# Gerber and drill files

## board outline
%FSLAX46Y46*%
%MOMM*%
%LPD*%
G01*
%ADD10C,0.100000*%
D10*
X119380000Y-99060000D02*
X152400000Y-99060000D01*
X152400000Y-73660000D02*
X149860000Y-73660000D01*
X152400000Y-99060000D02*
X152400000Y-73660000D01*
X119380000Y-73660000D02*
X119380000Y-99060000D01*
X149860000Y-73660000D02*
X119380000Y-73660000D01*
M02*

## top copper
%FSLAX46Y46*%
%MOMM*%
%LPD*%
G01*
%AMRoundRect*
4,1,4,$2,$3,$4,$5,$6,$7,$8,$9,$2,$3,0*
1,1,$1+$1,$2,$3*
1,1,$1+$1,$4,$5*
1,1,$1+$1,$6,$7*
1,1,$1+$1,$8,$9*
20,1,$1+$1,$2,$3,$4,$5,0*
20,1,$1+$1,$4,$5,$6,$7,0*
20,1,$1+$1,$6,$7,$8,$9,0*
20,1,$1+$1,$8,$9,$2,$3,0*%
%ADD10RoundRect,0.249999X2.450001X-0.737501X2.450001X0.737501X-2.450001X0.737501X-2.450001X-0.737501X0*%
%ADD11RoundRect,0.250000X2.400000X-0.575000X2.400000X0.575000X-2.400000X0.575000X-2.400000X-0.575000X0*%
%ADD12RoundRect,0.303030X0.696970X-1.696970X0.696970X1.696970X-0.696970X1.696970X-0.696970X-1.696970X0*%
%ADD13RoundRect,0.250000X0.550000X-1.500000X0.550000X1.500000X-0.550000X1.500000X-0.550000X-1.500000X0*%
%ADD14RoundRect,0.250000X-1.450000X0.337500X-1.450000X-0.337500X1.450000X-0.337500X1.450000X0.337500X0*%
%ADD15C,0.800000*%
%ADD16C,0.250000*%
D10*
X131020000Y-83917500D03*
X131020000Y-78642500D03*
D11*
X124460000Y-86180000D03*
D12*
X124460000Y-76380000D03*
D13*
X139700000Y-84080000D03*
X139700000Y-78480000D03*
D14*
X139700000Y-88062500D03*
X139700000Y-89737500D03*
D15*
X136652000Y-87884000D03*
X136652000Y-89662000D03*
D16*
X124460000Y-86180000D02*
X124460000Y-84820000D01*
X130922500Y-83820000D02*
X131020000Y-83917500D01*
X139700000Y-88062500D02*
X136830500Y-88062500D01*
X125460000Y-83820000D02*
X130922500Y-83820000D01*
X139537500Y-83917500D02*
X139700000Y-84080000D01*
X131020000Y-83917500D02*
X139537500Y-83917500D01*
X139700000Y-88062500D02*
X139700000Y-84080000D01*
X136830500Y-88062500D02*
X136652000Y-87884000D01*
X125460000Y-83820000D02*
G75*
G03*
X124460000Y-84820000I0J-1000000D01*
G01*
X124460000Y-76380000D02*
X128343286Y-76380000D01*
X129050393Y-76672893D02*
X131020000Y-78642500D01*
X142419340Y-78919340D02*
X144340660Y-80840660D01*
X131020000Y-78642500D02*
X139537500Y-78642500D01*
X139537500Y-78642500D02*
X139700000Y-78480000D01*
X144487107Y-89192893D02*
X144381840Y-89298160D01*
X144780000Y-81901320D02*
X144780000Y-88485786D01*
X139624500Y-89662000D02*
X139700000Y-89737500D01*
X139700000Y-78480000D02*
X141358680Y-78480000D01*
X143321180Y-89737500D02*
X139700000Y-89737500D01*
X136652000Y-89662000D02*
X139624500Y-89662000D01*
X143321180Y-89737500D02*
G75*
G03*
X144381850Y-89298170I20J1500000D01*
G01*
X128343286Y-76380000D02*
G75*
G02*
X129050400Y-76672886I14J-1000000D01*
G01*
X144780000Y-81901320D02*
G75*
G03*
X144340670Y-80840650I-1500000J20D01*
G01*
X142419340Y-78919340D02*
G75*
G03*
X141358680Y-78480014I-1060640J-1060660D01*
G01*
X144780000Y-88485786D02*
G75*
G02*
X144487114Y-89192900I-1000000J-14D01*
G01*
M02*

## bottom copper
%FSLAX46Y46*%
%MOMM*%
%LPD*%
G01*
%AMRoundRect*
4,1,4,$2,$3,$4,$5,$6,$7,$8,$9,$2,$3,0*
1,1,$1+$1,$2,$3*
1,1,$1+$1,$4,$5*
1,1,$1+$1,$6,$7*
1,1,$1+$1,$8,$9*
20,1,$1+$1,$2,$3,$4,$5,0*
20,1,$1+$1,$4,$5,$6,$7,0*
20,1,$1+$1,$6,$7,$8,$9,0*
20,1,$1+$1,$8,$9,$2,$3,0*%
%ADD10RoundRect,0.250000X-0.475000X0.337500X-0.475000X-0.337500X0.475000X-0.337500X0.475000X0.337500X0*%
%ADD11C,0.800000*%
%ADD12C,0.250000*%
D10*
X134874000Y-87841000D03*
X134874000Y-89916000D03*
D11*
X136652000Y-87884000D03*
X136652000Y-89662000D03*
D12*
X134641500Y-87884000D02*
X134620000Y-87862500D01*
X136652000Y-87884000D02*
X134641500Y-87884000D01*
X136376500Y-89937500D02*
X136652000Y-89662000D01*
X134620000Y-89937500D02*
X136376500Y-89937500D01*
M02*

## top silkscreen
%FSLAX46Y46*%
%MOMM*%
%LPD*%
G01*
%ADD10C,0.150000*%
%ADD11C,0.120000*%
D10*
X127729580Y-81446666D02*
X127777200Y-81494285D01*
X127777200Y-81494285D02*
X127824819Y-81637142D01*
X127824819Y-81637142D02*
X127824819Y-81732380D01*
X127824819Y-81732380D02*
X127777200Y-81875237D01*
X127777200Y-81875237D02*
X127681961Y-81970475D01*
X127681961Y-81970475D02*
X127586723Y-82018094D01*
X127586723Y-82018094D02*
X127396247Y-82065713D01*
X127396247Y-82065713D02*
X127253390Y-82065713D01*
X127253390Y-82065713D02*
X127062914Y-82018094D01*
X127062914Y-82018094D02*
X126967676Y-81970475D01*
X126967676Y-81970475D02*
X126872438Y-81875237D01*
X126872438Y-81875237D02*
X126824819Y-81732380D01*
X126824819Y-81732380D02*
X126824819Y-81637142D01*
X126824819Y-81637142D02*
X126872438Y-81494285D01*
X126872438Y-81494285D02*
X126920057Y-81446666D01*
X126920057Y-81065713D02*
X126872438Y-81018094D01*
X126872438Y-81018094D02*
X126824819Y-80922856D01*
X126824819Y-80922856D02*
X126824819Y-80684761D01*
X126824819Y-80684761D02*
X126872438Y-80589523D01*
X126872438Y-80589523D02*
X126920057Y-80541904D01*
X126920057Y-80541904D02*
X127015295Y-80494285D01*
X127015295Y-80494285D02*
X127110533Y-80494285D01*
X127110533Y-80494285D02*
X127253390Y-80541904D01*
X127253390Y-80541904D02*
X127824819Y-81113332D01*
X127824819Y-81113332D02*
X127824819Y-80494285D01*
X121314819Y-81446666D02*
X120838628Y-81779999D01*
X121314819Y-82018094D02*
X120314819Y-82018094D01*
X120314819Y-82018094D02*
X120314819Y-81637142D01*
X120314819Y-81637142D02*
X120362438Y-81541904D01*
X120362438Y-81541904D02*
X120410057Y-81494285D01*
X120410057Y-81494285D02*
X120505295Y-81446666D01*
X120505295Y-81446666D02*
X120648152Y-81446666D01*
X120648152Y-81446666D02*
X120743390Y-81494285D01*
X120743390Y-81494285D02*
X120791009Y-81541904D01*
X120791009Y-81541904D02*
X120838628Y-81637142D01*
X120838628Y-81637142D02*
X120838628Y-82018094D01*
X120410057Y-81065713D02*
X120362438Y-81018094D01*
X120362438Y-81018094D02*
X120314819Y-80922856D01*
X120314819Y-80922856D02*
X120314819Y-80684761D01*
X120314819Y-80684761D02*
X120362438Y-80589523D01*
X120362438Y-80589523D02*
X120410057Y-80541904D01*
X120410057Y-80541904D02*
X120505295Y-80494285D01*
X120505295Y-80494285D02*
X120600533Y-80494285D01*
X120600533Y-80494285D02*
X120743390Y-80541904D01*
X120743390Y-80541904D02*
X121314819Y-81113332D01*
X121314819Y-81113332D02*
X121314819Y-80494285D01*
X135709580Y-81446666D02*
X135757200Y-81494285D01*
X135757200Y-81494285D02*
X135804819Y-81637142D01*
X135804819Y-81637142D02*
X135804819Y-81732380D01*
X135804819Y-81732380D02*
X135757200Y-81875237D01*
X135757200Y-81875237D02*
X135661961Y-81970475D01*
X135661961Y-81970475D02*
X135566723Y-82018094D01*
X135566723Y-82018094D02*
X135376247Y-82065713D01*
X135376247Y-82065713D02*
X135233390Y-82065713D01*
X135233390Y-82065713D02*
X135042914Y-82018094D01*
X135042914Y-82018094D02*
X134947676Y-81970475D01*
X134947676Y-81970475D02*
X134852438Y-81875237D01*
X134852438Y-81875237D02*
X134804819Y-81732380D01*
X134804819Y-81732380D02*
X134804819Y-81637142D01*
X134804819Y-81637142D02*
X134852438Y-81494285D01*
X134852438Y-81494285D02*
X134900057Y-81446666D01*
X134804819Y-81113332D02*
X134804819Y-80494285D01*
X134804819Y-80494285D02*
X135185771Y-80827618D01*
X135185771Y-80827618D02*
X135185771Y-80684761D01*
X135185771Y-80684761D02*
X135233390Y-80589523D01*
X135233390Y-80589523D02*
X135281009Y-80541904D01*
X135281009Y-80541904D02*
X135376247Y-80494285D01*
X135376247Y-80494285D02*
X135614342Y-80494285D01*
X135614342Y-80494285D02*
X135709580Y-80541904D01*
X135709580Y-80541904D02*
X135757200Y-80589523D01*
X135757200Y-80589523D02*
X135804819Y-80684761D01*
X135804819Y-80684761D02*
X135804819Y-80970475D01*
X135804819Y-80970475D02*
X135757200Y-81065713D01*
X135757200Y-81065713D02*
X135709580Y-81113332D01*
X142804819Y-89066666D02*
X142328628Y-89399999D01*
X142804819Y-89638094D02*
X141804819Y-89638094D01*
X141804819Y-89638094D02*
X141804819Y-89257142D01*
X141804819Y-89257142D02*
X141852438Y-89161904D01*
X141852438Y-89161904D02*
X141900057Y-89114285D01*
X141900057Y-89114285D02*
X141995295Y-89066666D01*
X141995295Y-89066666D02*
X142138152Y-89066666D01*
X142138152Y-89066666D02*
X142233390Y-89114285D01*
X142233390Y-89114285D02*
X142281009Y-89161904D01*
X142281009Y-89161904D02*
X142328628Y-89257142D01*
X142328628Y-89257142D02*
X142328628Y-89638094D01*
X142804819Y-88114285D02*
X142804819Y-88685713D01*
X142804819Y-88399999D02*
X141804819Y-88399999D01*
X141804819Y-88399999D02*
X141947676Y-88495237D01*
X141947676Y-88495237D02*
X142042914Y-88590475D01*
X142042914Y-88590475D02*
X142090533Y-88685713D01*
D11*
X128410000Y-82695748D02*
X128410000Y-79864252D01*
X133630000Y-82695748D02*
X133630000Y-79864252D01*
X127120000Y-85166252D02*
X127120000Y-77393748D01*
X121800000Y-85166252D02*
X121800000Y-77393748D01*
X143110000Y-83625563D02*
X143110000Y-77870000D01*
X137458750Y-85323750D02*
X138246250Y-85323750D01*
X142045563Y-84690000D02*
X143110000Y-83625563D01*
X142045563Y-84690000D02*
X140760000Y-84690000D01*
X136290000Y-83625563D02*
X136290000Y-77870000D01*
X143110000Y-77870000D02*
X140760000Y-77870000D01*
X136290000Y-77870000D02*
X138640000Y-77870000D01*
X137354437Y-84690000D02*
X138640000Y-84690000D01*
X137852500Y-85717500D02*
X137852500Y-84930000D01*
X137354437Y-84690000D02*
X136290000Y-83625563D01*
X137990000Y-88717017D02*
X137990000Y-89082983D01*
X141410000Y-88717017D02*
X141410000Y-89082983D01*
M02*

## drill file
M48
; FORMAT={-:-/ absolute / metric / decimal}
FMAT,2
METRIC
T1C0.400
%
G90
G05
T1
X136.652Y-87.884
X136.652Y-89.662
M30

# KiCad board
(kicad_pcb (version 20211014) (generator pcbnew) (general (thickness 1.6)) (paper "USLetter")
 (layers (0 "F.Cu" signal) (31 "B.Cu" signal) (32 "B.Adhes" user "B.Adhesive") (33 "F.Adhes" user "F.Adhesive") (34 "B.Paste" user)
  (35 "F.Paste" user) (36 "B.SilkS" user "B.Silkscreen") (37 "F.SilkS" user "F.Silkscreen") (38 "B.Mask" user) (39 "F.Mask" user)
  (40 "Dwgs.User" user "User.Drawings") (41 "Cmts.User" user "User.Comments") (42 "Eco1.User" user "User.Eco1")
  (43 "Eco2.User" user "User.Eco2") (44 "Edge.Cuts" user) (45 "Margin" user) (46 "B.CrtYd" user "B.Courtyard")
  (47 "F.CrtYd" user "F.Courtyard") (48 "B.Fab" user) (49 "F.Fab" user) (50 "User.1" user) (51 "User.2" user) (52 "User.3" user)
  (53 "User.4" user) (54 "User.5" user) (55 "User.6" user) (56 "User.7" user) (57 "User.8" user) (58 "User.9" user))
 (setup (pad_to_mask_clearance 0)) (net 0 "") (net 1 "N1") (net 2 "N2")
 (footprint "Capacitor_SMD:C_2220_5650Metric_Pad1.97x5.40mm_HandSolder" (layer "F.Cu") (at 131.02 81.28 90)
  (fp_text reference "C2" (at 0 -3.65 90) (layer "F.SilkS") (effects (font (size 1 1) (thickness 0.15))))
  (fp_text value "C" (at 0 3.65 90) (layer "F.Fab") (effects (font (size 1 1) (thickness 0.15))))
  (fp_line (start -1.415748 -2.61) (end 1.415748 -2.61) (layer "F.SilkS") (width 0.12))
  (fp_line (start -1.415748 2.61) (end 1.415748 2.61) (layer "F.SilkS") (width 0.12))
  (pad "1" smd roundrect (at -2.6375 0 90) (size 1.975 5.4) (layers "F.Cu" "F.Paste" "F.Mask") (roundrect_rratio 0.126582) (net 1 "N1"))
  (pad "2" smd roundrect (at 2.6375 0 90) (size 1.975 5.4) (layers "F.Cu" "F.Paste" "F.Mask") (roundrect_rratio 0.126582) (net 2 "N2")))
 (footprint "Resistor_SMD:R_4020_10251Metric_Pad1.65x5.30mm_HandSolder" (layer "F.Cu") (at 124.46 81.28 90)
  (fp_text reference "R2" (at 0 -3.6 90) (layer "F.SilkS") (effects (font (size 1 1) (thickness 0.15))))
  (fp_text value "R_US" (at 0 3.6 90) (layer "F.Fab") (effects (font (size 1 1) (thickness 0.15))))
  (fp_line (start -3.886252 2.66) (end 3.886252 2.66) (layer "F.SilkS") (width 0.12))
  (fp_line (start -3.886252 -2.66) (end 3.886252 -2.66) (layer "F.SilkS") (width 0.12))
  (pad "1" smd roundrect (at -4.9 0 90) (size 1.65 5.3) (layers "F.Cu" "F.Paste" "F.Mask") (roundrect_rratio 0.151515) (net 1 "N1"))
  (pad "2" smd roundrect (at 4.9 0 90) (size 4 2) (layers "F.Cu" "F.Paste" "F.Mask") (roundrect_rratio 0.151515) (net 2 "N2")))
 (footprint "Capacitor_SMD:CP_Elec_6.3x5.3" (layer "F.Cu") (at 139.7 81.28 90)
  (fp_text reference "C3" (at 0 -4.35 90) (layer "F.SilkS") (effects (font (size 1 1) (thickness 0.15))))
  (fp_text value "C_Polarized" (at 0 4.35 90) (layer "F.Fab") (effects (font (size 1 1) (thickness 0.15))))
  (fp_line (start -2.345563 3.41) (end 3.41 3.41) (layer "F.SilkS") (width 0.12))
  (fp_line (start -4.04375 -2.24125) (end -4.04375 -1.45375) (layer "F.SilkS") (width 0.12))
  (fp_line (start -3.41 2.345563) (end -2.345563 3.41) (layer "F.SilkS") (width 0.12))
  (fp_line (start -3.41 2.345563) (end -3.41 1.06) (layer "F.SilkS") (width 0.12))
  (fp_line (start -2.345563 -3.41) (end 3.41 -3.41) (layer "F.SilkS") (width 0.12))
  (fp_line (start 3.41 3.41) (end 3.41 1.06) (layer "F.SilkS") (width 0.12))
  (fp_line (start 3.41 -3.41) (end 3.41 -1.06) (layer "F.SilkS") (width 0.12))
  (fp_line (start -3.41 -2.345563) (end -3.41 -1.06) (layer "F.SilkS") (width 0.12))
  (fp_line (start -4.4375 -1.8475) (end -3.65 -1.8475) (layer "F.SilkS") (width 0.12))
  (fp_line (start -3.41 -2.345563) (end -2.345563 -3.41) (layer "F.SilkS") (width 0.12))
  (pad "1" smd roundrect (at -2.8 0 90) (size 3.5 1.6) (layers "F.Cu" "F.Paste" "F.Mask") (roundrect_rratio 0.15625) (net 1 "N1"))
  (pad "2" smd roundrect (at 2.8 0 90) (size 3.5 1.6) (layers "F.Cu" "F.Paste" "F.Mask") (roundrect_rratio 0.15625) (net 2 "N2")))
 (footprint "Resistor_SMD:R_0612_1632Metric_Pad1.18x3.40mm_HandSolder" (layer "F.Cu") (at 139.7 88.9 -90)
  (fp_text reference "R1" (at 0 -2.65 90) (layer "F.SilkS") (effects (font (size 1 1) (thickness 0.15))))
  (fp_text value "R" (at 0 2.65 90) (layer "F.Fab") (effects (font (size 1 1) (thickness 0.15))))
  (fp_line (start -0.182983 1.71) (end 0.182983 1.71) (layer "F.SilkS") (width 0.12))
  (fp_line (start -0.182983 -1.71) (end 0.182983 -1.71) (layer "F.SilkS") (width 0.12))
  (pad "1" smd roundrect (at -0.8375 0 270) (size 1.175 3.4) (layers "F.Cu" "F.Paste" "F.Mask") (roundrect_rratio 0.212766) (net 1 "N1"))
  (pad "2" smd roundrect (at 0.8375 0 270) (size 1.175 3.4) (layers "F.Cu" "F.Paste" "F.Mask") (roundrect_rratio 0.212766) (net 2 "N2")))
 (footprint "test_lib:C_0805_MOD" (layer "B.Cu") (at 134.874 88.8785 -90)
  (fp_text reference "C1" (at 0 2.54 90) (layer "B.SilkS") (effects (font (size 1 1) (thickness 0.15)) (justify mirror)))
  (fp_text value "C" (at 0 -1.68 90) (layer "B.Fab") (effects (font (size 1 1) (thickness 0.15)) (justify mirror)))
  (pad "1" smd roundrect (at -1.0375 0 270) (size 1.175 1.45) (layers "B.Cu" "B.Paste" "B.Mask") (roundrect_rratio 0.212766) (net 1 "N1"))
  (pad "2" smd roundrect (at 1.0375 0 270) (size 1.175 1.45) (layers "B.Cu" "B.Paste" "B.Mask") (roundrect_rratio 0.212766) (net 2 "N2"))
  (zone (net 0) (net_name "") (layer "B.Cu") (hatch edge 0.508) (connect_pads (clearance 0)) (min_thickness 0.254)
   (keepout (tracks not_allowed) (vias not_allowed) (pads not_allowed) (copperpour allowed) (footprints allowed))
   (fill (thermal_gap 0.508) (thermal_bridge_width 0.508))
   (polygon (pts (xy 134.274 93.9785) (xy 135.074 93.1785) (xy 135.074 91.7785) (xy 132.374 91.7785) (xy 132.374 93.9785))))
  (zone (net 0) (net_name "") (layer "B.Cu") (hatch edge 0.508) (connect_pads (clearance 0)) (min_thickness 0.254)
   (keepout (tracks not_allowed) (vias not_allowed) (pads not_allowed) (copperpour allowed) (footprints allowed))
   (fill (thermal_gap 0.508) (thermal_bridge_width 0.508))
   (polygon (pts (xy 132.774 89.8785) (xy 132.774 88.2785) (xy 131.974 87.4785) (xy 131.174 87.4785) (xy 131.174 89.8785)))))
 (gr_line (start 119.38 99.06) (end 152.4 99.06) (layer "Edge.Cuts") (width 0.1))
 (gr_line (start 152.4 73.66) (end 149.86 73.66) (layer "Edge.Cuts") (width 0.1))
 (gr_line (start 152.4 99.06) (end 152.4 73.66) (layer "Edge.Cuts") (width 0.1))
 (gr_line (start 119.38 73.66) (end 119.38 99.06) (layer "Edge.Cuts") (width 0.1))
 (gr_line (start 149.86 73.66) (end 119.38 73.66) (layer "Edge.Cuts") (width 0.1))
 (segment (start 124.46 86.18) (end 124.46 84.82) (width 0.25) (layer "F.Cu") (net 1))
 (segment (start 130.9225 83.82) (end 131.02 83.9175) (width 0.25) (layer "F.Cu") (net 1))
 (segment (start 139.7 88.0625) (end 136.8305 88.0625) (width 0.25) (layer "F.Cu") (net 1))
 (segment (start 125.46 83.82) (end 130.9225 83.82) (width 0.25) (layer "F.Cu") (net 1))
 (segment (start 139.5375 83.9175) (end 139.7 84.08) (width 0.25) (layer "F.Cu") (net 1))
 (segment (start 131.02 83.9175) (end 139.5375 83.9175) (width 0.25) (layer "F.Cu") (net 1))
 (segment (start 139.7 88.0625) (end 139.7 84.08) (width 0.25) (layer "F.Cu") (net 1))
 (segment (start 136.8305 88.0625) (end 136.652 87.884) (width 0.25) (layer "F.Cu") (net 1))
 (via (at 136.652 87.884) (size 0.8) (drill 0.4) (layers "F.Cu" "B.Cu") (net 1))
 (arc (start 125.46 83.82) (mid 124.752893 84.112893) (end 124.46 84.82) (width 0.25) (layer "F.Cu") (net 1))
 (segment (start 134.6415 87.884) (end 134.62 87.8625) (width 0.25) (layer "B.Cu") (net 1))
 (segment (start 136.652 87.884) (end 134.6415 87.884) (width 0.25) (layer "B.Cu") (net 1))
 (segment (start 124.46 76.38) (end 128.343286 76.38) (width 0.25) (layer "F.Cu") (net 2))
 (segment (start 129.050393 76.672893) (end 131.02 78.6425) (width 0.25) (layer "F.Cu") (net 2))
 (segment (start 142.41934 78.91934) (end 144.34066 80.84066) (width 0.25) (layer "F.Cu") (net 2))
 (segment (start 131.02 78.6425) (end 139.5375 78.6425) (width 0.25) (layer "F.Cu") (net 2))
 (segment (start 139.5375 78.6425) (end 139.7 78.48) (width 0.25) (layer "F.Cu") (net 2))
 (segment (start 144.487107 89.192893) (end 144.38184 89.29816) (width 0.25) (layer "F.Cu") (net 2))
 (segment (start 144.78 81.90132) (end 144.78 88.485786) (width 0.25) (layer "F.Cu") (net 2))
 (segment (start 139.6245 89.662) (end 139.7 89.7375) (width 0.25) (layer "F.Cu") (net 2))
 (segment (start 139.7 78.48) (end 141.35868 78.48) (width 0.25) (layer "F.Cu") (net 2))
 (segment (start 143.32118 89.7375) (end 139.7 89.7375) (width 0.25) (layer "F.Cu") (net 2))
 (segment (start 136.652 89.662) (end 139.6245 89.662) (width 0.25) (layer "F.Cu") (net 2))
 (via (at 136.652 89.662) (size 0.8) (drill 0.4) (layers "F.Cu" "B.Cu") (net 2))
 (arc (start 143.32118 89.7375) (mid 143.895205 89.623319) (end 144.38184 89.29816) (width 0.25) (layer "F.Cu") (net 2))
 (arc (start 128.343286 76.38) (mid 128.725969 76.45612) (end 129.050393 76.672893) (width 0.25) (layer "F.Cu") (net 2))
 (arc (start 144.78 81.90132) (mid 144.665819 81.327295) (end 144.34066 80.84066) (width 0.25) (layer "F.Cu") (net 2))
 (arc (start 142.41934 78.91934) (mid 141.932705 78.594181) (end 141.35868 78.48) (width 0.25) (layer "F.Cu") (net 2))
 (arc (start 144.78 88.485786) (mid 144.70388 88.868469) (end 144.487107 89.192893) (width 0.25) (layer "F.Cu") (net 2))
 (segment (start 136.3765 89.9375) (end 136.652 89.662) (width 0.25) (layer "B.Cu") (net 2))
 (segment (start 134.62 89.9375) (end 136.3765 89.9375) (width 0.25) (layer "B.Cu") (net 2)))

